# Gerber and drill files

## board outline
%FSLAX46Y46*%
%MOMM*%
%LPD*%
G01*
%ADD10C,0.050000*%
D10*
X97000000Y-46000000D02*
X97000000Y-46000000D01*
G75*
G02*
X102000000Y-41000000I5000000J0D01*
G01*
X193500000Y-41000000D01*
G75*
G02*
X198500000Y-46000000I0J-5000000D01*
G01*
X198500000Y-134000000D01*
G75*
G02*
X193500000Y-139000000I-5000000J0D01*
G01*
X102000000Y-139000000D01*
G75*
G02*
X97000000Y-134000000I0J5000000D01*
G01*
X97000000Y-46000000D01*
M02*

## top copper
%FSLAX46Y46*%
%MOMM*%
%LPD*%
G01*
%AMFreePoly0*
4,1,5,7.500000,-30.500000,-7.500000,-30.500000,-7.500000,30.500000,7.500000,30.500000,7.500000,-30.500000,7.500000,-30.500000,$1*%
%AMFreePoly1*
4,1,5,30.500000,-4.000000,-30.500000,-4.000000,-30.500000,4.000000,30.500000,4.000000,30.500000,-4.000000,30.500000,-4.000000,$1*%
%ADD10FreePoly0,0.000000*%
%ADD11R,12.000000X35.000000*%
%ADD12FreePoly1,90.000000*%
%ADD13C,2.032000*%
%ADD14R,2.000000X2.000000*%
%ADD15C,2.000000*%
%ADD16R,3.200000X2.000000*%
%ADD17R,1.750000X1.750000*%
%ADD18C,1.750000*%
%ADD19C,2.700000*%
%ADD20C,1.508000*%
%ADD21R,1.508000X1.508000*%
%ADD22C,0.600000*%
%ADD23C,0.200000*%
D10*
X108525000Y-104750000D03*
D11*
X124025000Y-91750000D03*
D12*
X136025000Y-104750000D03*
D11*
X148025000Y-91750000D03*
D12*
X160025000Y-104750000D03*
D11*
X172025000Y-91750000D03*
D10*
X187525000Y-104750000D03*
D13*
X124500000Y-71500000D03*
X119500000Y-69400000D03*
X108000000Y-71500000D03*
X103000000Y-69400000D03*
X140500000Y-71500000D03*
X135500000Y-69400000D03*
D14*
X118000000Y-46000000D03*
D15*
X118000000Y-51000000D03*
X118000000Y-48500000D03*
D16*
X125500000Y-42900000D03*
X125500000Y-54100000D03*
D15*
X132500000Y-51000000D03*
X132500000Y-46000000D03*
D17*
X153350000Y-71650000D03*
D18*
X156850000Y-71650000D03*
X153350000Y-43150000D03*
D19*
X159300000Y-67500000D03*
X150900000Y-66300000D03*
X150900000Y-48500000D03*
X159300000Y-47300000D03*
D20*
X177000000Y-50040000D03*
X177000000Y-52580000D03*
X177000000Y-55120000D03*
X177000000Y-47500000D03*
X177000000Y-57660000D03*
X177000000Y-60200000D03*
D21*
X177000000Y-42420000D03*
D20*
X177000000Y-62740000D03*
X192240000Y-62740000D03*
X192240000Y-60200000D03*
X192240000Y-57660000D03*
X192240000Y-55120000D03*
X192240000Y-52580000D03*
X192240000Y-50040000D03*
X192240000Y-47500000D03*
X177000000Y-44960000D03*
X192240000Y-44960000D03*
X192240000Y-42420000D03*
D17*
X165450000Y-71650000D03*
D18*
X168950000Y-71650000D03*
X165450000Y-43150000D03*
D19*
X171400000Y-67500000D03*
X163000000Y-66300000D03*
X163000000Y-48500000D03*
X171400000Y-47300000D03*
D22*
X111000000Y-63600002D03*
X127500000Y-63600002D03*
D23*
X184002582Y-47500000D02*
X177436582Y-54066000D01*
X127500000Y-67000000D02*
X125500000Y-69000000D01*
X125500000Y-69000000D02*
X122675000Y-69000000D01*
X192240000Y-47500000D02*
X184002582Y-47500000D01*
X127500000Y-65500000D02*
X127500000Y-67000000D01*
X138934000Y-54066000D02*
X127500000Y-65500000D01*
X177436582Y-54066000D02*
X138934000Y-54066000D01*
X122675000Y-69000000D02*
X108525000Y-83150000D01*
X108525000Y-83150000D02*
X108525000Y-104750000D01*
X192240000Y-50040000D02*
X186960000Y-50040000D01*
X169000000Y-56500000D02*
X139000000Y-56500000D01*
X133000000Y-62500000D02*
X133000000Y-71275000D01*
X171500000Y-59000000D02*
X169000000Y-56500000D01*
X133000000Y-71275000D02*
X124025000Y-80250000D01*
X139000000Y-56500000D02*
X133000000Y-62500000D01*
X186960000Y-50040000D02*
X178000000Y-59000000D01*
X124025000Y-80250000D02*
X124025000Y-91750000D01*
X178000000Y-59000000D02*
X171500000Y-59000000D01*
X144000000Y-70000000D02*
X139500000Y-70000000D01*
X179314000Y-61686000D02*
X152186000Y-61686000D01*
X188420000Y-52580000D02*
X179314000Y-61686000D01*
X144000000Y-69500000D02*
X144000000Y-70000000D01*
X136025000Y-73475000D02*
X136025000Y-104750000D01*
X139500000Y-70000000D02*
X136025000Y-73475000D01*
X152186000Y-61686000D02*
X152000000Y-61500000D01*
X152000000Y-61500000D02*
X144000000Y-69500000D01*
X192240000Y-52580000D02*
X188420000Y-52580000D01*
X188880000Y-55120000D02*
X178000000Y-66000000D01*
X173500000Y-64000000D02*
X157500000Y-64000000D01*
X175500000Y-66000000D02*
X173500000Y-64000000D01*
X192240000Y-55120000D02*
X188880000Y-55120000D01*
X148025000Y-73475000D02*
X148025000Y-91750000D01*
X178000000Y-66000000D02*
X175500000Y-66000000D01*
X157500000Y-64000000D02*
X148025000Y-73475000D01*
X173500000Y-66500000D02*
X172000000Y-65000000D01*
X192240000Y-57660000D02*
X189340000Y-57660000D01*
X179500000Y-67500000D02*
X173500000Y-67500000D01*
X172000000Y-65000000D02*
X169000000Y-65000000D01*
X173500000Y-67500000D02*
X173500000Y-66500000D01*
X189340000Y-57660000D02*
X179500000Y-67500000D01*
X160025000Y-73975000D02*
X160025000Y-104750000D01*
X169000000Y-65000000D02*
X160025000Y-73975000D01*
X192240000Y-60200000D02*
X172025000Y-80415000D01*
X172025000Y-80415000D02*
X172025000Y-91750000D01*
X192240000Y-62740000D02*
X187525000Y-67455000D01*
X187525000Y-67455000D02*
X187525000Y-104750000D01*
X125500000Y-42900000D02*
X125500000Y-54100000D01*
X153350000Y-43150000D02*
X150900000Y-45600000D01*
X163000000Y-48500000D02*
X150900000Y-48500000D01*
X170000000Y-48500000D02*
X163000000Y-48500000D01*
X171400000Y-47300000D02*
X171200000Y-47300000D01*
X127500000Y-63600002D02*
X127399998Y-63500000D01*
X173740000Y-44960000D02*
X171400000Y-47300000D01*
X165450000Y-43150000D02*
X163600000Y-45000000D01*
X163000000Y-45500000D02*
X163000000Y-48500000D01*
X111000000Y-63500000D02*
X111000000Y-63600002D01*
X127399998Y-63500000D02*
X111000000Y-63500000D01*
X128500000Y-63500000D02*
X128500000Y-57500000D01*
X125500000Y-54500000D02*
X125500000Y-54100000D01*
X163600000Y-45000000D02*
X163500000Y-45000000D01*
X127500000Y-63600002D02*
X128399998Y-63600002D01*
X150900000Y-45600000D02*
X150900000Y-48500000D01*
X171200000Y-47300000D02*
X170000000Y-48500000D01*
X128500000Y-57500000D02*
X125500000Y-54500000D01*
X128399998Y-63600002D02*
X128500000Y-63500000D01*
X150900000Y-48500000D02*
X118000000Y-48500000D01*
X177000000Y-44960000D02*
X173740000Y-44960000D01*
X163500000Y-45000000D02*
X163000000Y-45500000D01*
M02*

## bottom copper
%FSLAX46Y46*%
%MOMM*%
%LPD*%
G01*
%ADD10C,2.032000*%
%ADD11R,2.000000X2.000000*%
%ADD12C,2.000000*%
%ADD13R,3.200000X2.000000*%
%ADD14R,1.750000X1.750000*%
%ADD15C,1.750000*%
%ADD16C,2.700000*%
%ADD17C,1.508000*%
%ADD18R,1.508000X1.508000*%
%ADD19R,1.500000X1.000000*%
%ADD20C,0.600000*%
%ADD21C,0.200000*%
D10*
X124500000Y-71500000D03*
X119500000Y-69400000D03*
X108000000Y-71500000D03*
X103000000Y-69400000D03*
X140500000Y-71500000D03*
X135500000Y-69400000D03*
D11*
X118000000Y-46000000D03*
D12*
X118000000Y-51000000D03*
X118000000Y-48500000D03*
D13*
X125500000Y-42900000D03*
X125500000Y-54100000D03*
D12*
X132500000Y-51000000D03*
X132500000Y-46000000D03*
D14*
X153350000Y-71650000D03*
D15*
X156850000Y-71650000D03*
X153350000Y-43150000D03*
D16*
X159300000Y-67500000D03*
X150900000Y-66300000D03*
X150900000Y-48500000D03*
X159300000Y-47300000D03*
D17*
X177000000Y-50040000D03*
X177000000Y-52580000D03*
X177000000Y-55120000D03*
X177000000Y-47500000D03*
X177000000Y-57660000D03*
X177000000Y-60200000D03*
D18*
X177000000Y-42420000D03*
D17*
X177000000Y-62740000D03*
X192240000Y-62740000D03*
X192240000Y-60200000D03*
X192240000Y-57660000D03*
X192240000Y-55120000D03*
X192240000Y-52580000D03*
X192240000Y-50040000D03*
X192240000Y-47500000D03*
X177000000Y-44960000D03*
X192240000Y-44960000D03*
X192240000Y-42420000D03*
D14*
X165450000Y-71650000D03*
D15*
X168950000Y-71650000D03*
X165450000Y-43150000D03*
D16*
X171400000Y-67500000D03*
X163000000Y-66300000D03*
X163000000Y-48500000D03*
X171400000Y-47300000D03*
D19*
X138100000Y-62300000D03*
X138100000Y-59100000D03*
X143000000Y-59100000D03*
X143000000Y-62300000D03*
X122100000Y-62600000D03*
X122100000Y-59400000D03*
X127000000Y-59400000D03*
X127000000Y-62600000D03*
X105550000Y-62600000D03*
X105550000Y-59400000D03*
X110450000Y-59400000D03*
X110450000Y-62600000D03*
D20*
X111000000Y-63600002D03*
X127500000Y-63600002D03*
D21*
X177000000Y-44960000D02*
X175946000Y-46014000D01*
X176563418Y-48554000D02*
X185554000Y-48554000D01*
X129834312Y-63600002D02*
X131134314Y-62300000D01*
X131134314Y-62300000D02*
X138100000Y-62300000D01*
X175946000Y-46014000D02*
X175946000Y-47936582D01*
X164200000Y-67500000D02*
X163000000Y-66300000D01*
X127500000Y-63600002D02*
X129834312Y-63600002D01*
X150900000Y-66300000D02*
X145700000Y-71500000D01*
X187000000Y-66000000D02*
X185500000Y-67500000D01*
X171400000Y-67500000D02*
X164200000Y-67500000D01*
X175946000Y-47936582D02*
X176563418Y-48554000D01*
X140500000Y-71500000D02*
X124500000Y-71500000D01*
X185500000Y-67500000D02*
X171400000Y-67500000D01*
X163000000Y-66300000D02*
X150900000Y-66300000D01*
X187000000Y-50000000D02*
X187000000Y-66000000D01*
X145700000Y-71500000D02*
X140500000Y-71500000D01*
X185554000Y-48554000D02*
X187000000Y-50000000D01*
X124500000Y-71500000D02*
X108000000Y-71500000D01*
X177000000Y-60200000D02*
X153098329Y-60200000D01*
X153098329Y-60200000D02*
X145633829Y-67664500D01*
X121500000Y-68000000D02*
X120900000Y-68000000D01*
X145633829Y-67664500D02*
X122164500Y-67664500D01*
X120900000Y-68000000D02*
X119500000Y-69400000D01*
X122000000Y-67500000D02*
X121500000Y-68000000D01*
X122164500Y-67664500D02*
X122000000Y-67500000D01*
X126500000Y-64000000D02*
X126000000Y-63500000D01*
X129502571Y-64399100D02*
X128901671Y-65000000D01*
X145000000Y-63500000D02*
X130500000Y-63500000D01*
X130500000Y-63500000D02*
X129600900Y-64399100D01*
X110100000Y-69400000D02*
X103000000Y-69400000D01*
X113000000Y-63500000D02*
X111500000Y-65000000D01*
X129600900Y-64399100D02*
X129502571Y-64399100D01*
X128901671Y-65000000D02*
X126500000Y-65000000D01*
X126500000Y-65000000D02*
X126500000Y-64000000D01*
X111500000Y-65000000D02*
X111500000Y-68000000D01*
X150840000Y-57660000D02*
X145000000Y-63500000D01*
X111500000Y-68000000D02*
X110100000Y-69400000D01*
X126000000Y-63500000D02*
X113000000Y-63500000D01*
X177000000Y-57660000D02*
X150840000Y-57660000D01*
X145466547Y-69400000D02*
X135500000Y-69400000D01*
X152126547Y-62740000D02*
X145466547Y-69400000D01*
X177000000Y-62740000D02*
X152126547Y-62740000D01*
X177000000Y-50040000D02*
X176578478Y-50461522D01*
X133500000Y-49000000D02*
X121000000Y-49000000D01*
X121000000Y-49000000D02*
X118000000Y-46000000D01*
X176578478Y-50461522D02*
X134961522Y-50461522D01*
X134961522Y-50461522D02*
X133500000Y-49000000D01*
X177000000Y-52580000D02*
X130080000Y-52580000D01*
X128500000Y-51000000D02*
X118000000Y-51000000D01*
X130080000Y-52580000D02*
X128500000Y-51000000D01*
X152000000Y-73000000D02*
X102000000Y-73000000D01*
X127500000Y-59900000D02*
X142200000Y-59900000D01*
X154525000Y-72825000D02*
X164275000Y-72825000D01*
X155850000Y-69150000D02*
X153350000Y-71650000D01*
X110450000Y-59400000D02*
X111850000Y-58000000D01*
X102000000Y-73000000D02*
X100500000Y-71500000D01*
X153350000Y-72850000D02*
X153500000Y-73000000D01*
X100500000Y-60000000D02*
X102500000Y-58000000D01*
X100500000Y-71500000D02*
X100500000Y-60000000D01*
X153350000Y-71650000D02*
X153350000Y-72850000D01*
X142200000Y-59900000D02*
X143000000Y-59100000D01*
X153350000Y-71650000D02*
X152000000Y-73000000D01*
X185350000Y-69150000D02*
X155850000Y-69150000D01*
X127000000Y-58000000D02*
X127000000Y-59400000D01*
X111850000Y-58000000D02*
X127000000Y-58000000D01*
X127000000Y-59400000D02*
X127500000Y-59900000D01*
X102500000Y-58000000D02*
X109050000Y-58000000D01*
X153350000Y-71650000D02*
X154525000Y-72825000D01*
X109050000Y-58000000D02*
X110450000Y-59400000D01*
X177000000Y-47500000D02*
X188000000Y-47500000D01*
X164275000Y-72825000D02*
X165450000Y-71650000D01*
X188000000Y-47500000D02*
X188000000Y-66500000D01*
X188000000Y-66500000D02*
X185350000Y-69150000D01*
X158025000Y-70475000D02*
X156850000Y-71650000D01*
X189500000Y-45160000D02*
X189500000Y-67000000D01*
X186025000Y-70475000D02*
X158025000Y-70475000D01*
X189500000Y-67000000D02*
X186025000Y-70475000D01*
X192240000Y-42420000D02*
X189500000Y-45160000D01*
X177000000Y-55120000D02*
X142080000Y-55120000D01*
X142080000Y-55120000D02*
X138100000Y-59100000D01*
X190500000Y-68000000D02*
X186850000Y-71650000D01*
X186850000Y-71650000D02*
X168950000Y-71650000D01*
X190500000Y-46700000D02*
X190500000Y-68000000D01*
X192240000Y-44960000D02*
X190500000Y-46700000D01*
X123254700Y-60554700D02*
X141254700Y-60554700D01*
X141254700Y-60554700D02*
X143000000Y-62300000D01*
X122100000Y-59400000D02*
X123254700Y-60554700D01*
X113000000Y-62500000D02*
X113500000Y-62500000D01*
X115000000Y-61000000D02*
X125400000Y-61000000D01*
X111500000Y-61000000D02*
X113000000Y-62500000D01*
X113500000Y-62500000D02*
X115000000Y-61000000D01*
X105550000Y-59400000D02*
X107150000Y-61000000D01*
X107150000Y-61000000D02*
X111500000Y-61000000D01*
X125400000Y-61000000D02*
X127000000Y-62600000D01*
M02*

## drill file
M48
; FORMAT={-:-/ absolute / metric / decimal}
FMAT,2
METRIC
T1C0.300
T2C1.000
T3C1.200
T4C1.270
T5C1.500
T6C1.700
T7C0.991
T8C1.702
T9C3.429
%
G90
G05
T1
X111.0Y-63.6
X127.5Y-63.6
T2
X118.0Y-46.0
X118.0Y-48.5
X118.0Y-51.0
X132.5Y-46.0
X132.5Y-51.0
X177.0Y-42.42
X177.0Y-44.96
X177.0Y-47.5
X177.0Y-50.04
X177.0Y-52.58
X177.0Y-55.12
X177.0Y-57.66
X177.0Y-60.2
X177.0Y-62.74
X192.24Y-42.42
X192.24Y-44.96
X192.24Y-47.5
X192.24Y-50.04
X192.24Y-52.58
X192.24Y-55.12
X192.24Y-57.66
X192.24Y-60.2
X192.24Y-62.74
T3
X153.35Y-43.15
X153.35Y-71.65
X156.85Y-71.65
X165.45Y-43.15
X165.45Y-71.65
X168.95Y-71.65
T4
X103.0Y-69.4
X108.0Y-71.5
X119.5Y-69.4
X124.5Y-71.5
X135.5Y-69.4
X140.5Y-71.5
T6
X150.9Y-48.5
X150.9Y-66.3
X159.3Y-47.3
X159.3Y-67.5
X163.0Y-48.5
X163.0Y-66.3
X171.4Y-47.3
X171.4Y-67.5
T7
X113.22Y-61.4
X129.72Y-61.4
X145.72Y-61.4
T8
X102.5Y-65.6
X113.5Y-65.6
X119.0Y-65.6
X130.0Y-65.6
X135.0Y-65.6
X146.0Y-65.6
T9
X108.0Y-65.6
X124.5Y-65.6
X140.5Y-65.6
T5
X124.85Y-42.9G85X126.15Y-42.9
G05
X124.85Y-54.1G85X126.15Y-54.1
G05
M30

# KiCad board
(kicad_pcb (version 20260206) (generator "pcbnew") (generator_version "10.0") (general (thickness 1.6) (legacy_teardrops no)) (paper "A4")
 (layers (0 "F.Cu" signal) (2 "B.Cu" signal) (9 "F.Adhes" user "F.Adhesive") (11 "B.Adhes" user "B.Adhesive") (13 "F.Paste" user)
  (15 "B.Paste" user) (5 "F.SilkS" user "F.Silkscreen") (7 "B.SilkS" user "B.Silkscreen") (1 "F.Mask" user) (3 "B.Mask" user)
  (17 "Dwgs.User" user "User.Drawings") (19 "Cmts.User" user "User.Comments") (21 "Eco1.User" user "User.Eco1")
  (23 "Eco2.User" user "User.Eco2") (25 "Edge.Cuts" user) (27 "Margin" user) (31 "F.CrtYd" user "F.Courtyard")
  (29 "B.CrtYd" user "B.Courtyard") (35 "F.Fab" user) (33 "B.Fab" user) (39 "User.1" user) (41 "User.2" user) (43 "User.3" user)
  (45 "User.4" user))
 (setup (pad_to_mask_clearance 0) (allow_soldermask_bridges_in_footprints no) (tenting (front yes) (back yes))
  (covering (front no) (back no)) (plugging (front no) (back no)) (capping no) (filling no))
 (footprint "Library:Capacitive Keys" (layer "F.Cu") (at 139.025 60.25)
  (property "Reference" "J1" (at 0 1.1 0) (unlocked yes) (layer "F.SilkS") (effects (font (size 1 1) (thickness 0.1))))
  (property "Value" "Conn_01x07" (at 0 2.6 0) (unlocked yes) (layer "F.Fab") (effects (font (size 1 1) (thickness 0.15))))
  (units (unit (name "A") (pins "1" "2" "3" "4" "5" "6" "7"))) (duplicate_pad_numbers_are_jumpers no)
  (pad "1" smd custom (at -30.5 44.5) (size 15 61) (layers "F.Cu" "F.Mask") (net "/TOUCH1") (options (clearance outline) (anchor rect))
   (primitives))
  (pad "2" smd rect (at -15 31.5) (size 12 35) (layers "F.Cu" "F.Mask") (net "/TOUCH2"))
  (pad "3" smd custom (at -3 44.5 90) (size 61 8) (layers "F.Cu" "F.Mask") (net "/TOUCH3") (options (clearance outline) (anchor rect))
   (primitives))
  (pad "4" smd rect (at 9 31.5) (size 12 35) (layers "F.Cu" "F.Mask") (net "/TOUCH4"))
  (pad "5" smd custom (at 21 44.5 90) (size 61 8) (layers "F.Cu" "F.Mask") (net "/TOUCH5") (options (clearance outline) (anchor rect))
   (primitives))
  (pad "6" smd rect (at 33 31.5) (size 12 35) (layers "F.Cu" "F.Mask") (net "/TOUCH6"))
  (pad "7" smd custom (at 48.5 44.5) (size 15 61) (layers "F.Cu" "F.Mask") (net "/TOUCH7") (options (clearance outline) (anchor rect))
   (primitives)))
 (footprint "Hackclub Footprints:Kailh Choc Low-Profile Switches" (layer "F.Cu") (at 124.5 65.6)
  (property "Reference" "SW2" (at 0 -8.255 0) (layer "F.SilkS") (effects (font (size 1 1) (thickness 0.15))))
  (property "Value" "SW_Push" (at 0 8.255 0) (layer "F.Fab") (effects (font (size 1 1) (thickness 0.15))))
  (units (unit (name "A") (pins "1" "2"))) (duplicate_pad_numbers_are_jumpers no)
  (pad "" np_thru_hole circle (at -5.5 0) (size 1.7018 1.7018) (drill 1.7018) (layers "*.Cu" "*.Mask"))
  (pad "" np_thru_hole circle (at 0 0) (size 3.429 3.429) (drill 3.429) (layers "*.Cu" "*.Mask"))
  (pad "" np_thru_hole circle (at 5.22 -4.2) (size 0.9906 0.9906) (drill 0.9906) (layers "*.Cu" "*.Mask"))
  (pad "" np_thru_hole circle (at 5.5 0) (size 1.7018 1.7018) (drill 1.7018) (layers "*.Cu" "*.Mask"))
  (pad "1" thru_hole circle (at 0 5.9) (size 2.032 2.032) (drill 1.27) (layers "*.Cu" "*.Mask") (remove_unused_layers no) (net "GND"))
  (pad "2" thru_hole circle (at -5 3.8) (size 2.032 2.032) (drill 1.27) (layers "*.Cu" "*.Mask") (remove_unused_layers no) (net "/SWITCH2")))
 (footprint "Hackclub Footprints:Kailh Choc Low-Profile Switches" (layer "F.Cu") (at 108 65.6)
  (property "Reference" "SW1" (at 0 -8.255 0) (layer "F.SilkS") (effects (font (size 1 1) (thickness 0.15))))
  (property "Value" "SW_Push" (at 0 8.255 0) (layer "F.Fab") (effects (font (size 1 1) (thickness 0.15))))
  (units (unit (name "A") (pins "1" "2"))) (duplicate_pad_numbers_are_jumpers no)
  (pad "" np_thru_hole circle (at -5.5 0) (size 1.7018 1.7018) (drill 1.7018) (layers "*.Cu" "*.Mask"))
  (pad "" np_thru_hole circle (at 0 0) (size 3.429 3.429) (drill 3.429) (layers "*.Cu" "*.Mask"))
  (pad "" np_thru_hole circle (at 5.22 -4.2) (size 0.9906 0.9906) (drill 0.9906) (layers "*.Cu" "*.Mask"))
  (pad "" np_thru_hole circle (at 5.5 0) (size 1.7018 1.7018) (drill 1.7018) (layers "*.Cu" "*.Mask"))
  (pad "1" thru_hole circle (at 0 5.9) (size 2.032 2.032) (drill 1.27) (layers "*.Cu" "*.Mask") (remove_unused_layers no) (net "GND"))
  (pad "2" thru_hole circle (at -5 3.8) (size 2.032 2.032) (drill 1.27) (layers "*.Cu" "*.Mask") (remove_unused_layers no) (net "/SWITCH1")))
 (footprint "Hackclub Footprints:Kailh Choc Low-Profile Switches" (layer "F.Cu") (at 140.5 65.6)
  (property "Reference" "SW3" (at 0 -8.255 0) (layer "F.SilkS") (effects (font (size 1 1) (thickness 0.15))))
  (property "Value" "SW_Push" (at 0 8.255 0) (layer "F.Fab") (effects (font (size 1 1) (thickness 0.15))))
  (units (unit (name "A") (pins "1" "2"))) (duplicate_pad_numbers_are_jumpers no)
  (pad "" np_thru_hole circle (at -5.5 0) (size 1.7018 1.7018) (drill 1.7018) (layers "*.Cu" "*.Mask"))
  (pad "" np_thru_hole circle (at 0 0) (size 3.429 3.429) (drill 3.429) (layers "*.Cu" "*.Mask"))
  (pad "" np_thru_hole circle (at 5.22 -4.2) (size 0.9906 0.9906) (drill 0.9906) (layers "*.Cu" "*.Mask"))
  (pad "" np_thru_hole circle (at 5.5 0) (size 1.7018 1.7018) (drill 1.7018) (layers "*.Cu" "*.Mask"))
  (pad "1" thru_hole circle (at 0 5.9) (size 2.032 2.032) (drill 1.27) (layers "*.Cu" "*.Mask") (remove_unused_layers no) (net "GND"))
  (pad "2" thru_hole circle (at -5 3.8) (size 2.032 2.032) (drill 1.27) (layers "*.Cu" "*.Mask") (remove_unused_layers no) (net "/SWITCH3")))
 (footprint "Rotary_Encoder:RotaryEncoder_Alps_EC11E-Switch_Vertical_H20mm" (layer "F.Cu") (at 118 46)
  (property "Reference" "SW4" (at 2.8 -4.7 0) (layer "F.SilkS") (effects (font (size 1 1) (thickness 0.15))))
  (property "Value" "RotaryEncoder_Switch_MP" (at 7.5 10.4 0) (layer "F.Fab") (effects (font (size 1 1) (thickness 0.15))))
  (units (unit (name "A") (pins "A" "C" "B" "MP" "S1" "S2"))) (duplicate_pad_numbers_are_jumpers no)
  (pad "A" thru_hole rect (at 0 0) (size 2 2) (drill 1) (layers "*.Cu" "*.Mask") (remove_unused_layers no) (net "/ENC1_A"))
  (pad "B" thru_hole circle (at 0 5) (size 2 2) (drill 1) (layers "*.Cu" "*.Mask") (remove_unused_layers no) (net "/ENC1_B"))
  (pad "C" thru_hole circle (at 0 2.5) (size 2 2) (drill 1) (layers "*.Cu" "*.Mask") (remove_unused_layers no) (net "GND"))
  (pad "MP" thru_hole rect (at 7.5 -3.1) (size 3.2 2) (drill oval 2.8 1.5) (layers "*.Cu" "*.Mask") (remove_unused_layers no) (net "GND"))
  (pad "MP" thru_hole rect (at 7.5 8.1) (size 3.2 2) (drill oval 2.8 1.5) (layers "*.Cu" "*.Mask") (remove_unused_layers no) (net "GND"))
  (pad "S1" thru_hole circle (at 14.5 5) (size 2 2) (drill 1) (layers "*.Cu" "*.Mask") (remove_unused_layers no)
   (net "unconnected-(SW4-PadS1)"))
  (pad "S2" thru_hole circle (at 14.5 0) (size 2 2) (drill 1) (layers "*.Cu" "*.Mask") (remove_unused_layers no)
   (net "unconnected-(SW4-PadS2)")))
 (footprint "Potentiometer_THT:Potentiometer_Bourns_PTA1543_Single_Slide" (layer "F.Cu") (at 153.35 71.65 90)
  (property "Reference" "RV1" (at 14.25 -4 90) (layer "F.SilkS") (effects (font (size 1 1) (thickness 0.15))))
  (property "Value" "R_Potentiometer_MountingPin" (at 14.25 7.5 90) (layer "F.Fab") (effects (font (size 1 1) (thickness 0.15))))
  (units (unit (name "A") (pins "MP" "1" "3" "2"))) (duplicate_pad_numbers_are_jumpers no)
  (pad "1" thru_hole rect (at 0 0 90) (size 1.75 1.75) (drill 1.2) (layers "*.Cu" "*.Mask") (remove_unused_layers no) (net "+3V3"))
  (pad "2" thru_hole circle (at 0 3.5 90) (size 1.75 1.75) (drill 1.2) (layers "*.Cu" "*.Mask") (remove_unused_layers no) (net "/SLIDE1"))
  (pad "3" thru_hole circle (at 28.5 0 90) (size 1.75 1.75) (drill 1.2) (layers "*.Cu" "*.Mask") (remove_unused_layers no) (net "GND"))
  (pad "MP" thru_hole circle (at 4.15 5.95 90) (size 2.7 2.7) (drill 1.7) (layers "*.Cu" "*.Mask") (remove_unused_layers no) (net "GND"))
  (pad "MP" thru_hole circle (at 5.35 -2.45 90) (size 2.7 2.7) (drill 1.7) (layers "*.Cu" "*.Mask") (remove_unused_layers no) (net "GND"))
  (pad "MP" thru_hole circle (at 23.15 -2.45 90) (size 2.7 2.7) (drill 1.7) (layers "*.Cu" "*.Mask") (remove_unused_layers no) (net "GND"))
  (pad "MP" thru_hole circle (at 24.35 5.95 90) (size 2.7 2.7) (drill 1.7) (layers "*.Cu" "*.Mask") (remove_unused_layers no) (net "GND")))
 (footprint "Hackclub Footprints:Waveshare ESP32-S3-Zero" (layer "F.Cu") (at 184.62 52.58)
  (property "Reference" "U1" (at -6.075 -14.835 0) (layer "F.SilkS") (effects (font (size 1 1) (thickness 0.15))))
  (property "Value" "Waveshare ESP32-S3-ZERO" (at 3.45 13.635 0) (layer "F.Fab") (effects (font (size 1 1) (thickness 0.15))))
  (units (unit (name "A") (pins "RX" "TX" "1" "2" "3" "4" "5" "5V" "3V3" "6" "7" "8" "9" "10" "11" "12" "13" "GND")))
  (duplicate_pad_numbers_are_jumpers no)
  (pad "1" thru_hole circle (at -7.62 -2.54) (size 1.508 1.508) (drill 1) (layers "*.Cu" "*.Mask") (remove_unused_layers no) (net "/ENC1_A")
   (solder_mask_margin 0.102))
  (pad "2" thru_hole circle (at -7.62 0) (size 1.508 1.508) (drill 1) (layers "*.Cu" "*.Mask") (remove_unused_layers no) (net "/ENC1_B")
   (solder_mask_margin 0.102))
  (pad "3" thru_hole circle (at -7.62 2.54) (size 1.508 1.508) (drill 1) (layers "*.Cu" "*.Mask") (remove_unused_layers no) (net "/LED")
   (solder_mask_margin 0.102))
  (pad "3V3" thru_hole circle (at -7.62 -5.08) (size 1.508 1.508) (drill 1) (layers "*.Cu" "*.Mask") (remove_unused_layers no) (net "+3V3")
   (solder_mask_margin 0.102))
  (pad "4" thru_hole circle (at -7.62 5.08) (size 1.508 1.508) (drill 1) (layers "*.Cu" "*.Mask") (remove_unused_layers no) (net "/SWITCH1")
   (solder_mask_margin 0.102))
  (pad "5" thru_hole circle (at -7.62 7.62) (size 1.508 1.508) (drill 1) (layers "*.Cu" "*.Mask") (remove_unused_layers no) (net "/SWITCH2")
   (solder_mask_margin 0.102))
  (pad "5V" thru_hole rect (at -7.62 -10.16) (size 1.508 1.508) (drill 1) (layers "*.Cu" "*.Mask") (remove_unused_layers no) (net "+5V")
   (solder_mask_margin 0.102))
  (pad "6" thru_hole circle (at -7.62 10.16) (size 1.508 1.508) (drill 1) (layers "*.Cu" "*.Mask") (remove_unused_layers no)
   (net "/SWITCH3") (solder_mask_margin 0.102))
  (pad "7" thru_hole circle (at 7.62 10.16) (size 1.508 1.508) (drill 1) (layers "*.Cu" "*.Mask") (remove_unused_layers no) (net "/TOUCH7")
   (solder_mask_margin 0.102))
  (pad "8" thru_hole circle (at 7.62 7.62) (size 1.508 1.508) (drill 1) (layers "*.Cu" "*.Mask") (remove_unused_layers no) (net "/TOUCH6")
   (solder_mask_margin 0.102))
  (pad "9" thru_hole circle (at 7.62 5.08) (size 1.508 1.508) (drill 1) (layers "*.Cu" "*.Mask") (remove_unused_layers no) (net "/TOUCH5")
   (solder_mask_margin 0.102))
  (pad "10" thru_hole circle (at 7.62 2.54) (size 1.508 1.508) (drill 1) (layers "*.Cu" "*.Mask") (remove_unused_layers no) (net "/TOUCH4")
   (solder_mask_margin 0.102))
  (pad "11" thru_hole circle (at 7.62 0) (size 1.508 1.508) (drill 1) (layers "*.Cu" "*.Mask") (remove_unused_layers no) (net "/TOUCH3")
   (solder_mask_margin 0.102))
  (pad "12" thru_hole circle (at 7.62 -2.54) (size 1.508 1.508) (drill 1) (layers "*.Cu" "*.Mask") (remove_unused_layers no) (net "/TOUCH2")
   (solder_mask_margin 0.102))
  (pad "13" thru_hole circle (at 7.62 -5.08) (size 1.508 1.508) (drill 1) (layers "*.Cu" "*.Mask") (remove_unused_layers no) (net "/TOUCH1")
   (solder_mask_margin 0.102))
  (pad "GND" thru_hole circle (at -7.62 -7.62) (size 1.508 1.508) (drill 1) (layers "*.Cu" "*.Mask") (remove_unused_layers no) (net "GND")
   (solder_mask_margin 0.102))
  (pad "RX" thru_hole circle (at 7.62 -7.62) (size 1.508 1.508) (drill 1) (layers "*.Cu" "*.Mask") (remove_unused_layers no) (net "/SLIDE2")
   (solder_mask_margin 0.102))
  (pad "TX" thru_hole circle (at 7.62 -10.16) (size 1.508 1.508) (drill 1) (layers "*.Cu" "*.Mask") (remove_unused_layers no)
   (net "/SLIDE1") (solder_mask_margin 0.102)))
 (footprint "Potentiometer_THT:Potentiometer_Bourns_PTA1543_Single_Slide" (layer "F.Cu") (at 165.45 71.65 90)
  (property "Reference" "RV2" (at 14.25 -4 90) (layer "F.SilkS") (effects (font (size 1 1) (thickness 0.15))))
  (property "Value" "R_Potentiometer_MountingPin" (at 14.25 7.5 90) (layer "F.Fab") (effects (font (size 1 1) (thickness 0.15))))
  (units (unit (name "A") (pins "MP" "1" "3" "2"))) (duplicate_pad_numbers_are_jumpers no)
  (pad "1" thru_hole rect (at 0 0 90) (size 1.75 1.75) (drill 1.2) (layers "*.Cu" "*.Mask") (remove_unused_layers no) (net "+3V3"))
  (pad "2" thru_hole circle (at 0 3.5 90) (size 1.75 1.75) (drill 1.2) (layers "*.Cu" "*.Mask") (remove_unused_layers no) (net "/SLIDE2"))
  (pad "3" thru_hole circle (at 28.5 0 90) (size 1.75 1.75) (drill 1.2) (layers "*.Cu" "*.Mask") (remove_unused_layers no) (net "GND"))
  (pad "MP" thru_hole circle (at 4.15 5.95 90) (size 2.7 2.7) (drill 1.7) (layers "*.Cu" "*.Mask") (remove_unused_layers no) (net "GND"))
  (pad "MP" thru_hole circle (at 5.35 -2.45 90) (size 2.7 2.7) (drill 1.7) (layers "*.Cu" "*.Mask") (remove_unused_layers no) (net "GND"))
  (pad "MP" thru_hole circle (at 23.15 -2.45 90) (size 2.7 2.7) (drill 1.7) (layers "*.Cu" "*.Mask") (remove_unused_layers no) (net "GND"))
  (pad "MP" thru_hole circle (at 24.35 5.95 90) (size 2.7 2.7) (drill 1.7) (layers "*.Cu" "*.Mask") (remove_unused_layers no) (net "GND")))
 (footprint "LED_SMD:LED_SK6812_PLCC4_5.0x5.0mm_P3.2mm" (layer "B.Cu") (at 140.55 60.7)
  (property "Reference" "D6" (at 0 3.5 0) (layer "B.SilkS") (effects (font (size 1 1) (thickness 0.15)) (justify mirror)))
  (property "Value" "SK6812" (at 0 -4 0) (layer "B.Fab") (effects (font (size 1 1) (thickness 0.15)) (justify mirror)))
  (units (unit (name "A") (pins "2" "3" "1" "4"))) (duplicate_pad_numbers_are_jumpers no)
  (pad "1" smd rect (at -2.45 1.6 180) (size 1.5 1) (layers "B.Cu" "B.Mask" "B.Paste") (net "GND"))
  (pad "2" smd rect (at -2.45 -1.6 180) (size 1.5 1) (layers "B.Cu" "B.Mask" "B.Paste") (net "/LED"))
  (pad "3" smd rect (at 2.45 -1.6 180) (size 1.5 1) (layers "B.Cu" "B.Mask" "B.Paste") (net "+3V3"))
  (pad "4" smd rect (at 2.45 1.6 180) (size 1.5 1) (layers "B.Cu" "B.Mask" "B.Paste") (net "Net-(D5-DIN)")))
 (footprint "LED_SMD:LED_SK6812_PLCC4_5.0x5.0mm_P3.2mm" (layer "B.Cu") (at 124.55 61)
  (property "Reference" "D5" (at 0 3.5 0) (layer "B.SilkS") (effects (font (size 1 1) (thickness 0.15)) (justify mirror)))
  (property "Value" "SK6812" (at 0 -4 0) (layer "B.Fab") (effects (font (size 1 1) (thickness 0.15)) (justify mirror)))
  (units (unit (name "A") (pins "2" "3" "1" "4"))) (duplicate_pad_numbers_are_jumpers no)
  (pad "1" smd rect (at -2.45 1.6 180) (size 1.5 1) (layers "B.Cu" "B.Mask" "B.Paste") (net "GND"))
  (pad "2" smd rect (at -2.45 -1.6 180) (size 1.5 1) (layers "B.Cu" "B.Mask" "B.Paste") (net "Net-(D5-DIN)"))
  (pad "3" smd rect (at 2.45 -1.6 180) (size 1.5 1) (layers "B.Cu" "B.Mask" "B.Paste") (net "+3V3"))
  (pad "4" smd rect (at 2.45 1.6 180) (size 1.5 1) (layers "B.Cu" "B.Mask" "B.Paste") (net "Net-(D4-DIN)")))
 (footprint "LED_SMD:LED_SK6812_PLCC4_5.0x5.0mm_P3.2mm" (layer "B.Cu") (at 108 61)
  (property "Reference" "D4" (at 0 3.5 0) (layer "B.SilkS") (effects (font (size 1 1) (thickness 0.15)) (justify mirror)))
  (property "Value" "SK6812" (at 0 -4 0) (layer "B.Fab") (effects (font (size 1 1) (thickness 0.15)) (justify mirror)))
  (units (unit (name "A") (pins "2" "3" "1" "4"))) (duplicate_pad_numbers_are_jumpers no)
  (pad "1" smd rect (at -2.45 1.6 180) (size 1.5 1) (layers "B.Cu" "B.Mask" "B.Paste") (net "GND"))
  (pad "2" smd rect (at -2.45 -1.6 180) (size 1.5 1) (layers "B.Cu" "B.Mask" "B.Paste") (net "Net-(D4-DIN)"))
  (pad "3" smd rect (at 2.45 -1.6 180) (size 1.5 1) (layers "B.Cu" "B.Mask" "B.Paste") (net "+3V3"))
  (pad "4" smd rect (at 2.45 1.6 180) (size 1.5 1) (layers "B.Cu" "B.Mask" "B.Paste") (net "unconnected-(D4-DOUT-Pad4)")))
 (gr_rect (start 97 41) (end 198.5 139) (radius 5) (stroke (width 0.05) (type solid)) (fill no) (layer "Edge.Cuts"))
 (segment (start 184.002582 47.5) (end 177.436582 54.066) (width 0.2) (layer "F.Cu") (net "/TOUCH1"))
 (segment (start 127.5 67) (end 125.5 69) (width 0.2) (layer "F.Cu") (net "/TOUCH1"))
 (segment (start 125.5 69) (end 122.675 69) (width 0.2) (layer "F.Cu") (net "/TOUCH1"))
 (segment (start 192.24 47.5) (end 184.002582 47.5) (width 0.2) (layer "F.Cu") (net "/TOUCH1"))
 (segment (start 127.5 65.5) (end 127.5 67) (width 0.2) (layer "F.Cu") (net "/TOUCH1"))
 (segment (start 138.934 54.066) (end 127.5 65.5) (width 0.2) (layer "F.Cu") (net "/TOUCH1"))
 (segment (start 177.436582 54.066) (end 138.934 54.066) (width 0.2) (layer "F.Cu") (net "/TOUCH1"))
 (segment (start 122.675 69) (end 108.525 83.15) (width 0.2) (layer "F.Cu") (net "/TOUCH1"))
 (segment (start 108.525 83.15) (end 108.525 104.75) (width 0.2) (layer "F.Cu") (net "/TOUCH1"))
 (segment (start 192.24 50.04) (end 186.96 50.04) (width 0.2) (layer "F.Cu") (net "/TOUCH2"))
 (segment (start 169 56.5) (end 139 56.5) (width 0.2) (layer "F.Cu") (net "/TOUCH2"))
 (segment (start 133 62.5) (end 133 71.275) (width 0.2) (layer "F.Cu") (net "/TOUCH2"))
 (segment (start 171.5 59) (end 169 56.5) (width 0.2) (layer "F.Cu") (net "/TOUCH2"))
 (segment (start 133 71.275) (end 124.025 80.25) (width 0.2) (layer "F.Cu") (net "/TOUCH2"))
 (segment (start 139 56.5) (end 133 62.5) (width 0.2) (layer "F.Cu") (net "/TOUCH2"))
 (segment (start 186.96 50.04) (end 178 59) (width 0.2) (layer "F.Cu") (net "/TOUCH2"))
 (segment (start 124.025 80.25) (end 124.025 91.75) (width 0.2) (layer "F.Cu") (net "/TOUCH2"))
 (segment (start 178 59) (end 171.5 59) (width 0.2) (layer "F.Cu") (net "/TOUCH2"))
 (segment (start 144 70) (end 139.5 70) (width 0.2) (layer "F.Cu") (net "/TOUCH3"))
 (segment (start 179.314 61.686) (end 152.186 61.686) (width 0.2) (layer "F.Cu") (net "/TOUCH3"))
 (segment (start 188.42 52.58) (end 179.314 61.686) (width 0.2) (layer "F.Cu") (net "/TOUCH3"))
 (segment (start 144 69.5) (end 144 70) (width 0.2) (layer "F.Cu") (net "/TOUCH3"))
 (segment (start 136.025 73.475) (end 136.025 104.75) (width 0.2) (layer "F.Cu") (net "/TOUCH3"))
 (segment (start 139.5 70) (end 136.025 73.475) (width 0.2) (layer "F.Cu") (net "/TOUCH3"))
 (segment (start 152.186 61.686) (end 152 61.5) (width 0.2) (layer "F.Cu") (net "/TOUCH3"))
 (segment (start 152 61.5) (end 144 69.5) (width 0.2) (layer "F.Cu") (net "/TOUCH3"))
 (segment (start 192.24 52.58) (end 188.42 52.58) (width 0.2) (layer "F.Cu") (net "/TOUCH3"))
 (segment (start 188.88 55.12) (end 178 66) (width 0.2) (layer "F.Cu") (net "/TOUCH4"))
 (segment (start 173.5 64) (end 157.5 64) (width 0.2) (layer "F.Cu") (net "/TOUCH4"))
 (segment (start 175.5 66) (end 173.5 64) (width 0.2) (layer "F.Cu") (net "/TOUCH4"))
 (segment (start 192.24 55.12) (end 188.88 55.12) (width 0.2) (layer "F.Cu") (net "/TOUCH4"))
 (segment (start 148.025 73.475) (end 148.025 91.75) (width 0.2) (layer "F.Cu") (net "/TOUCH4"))
 (segment (start 178 66) (end 175.5 66) (width 0.2) (layer "F.Cu") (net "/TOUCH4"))
 (segment (start 157.5 64) (end 148.025 73.475) (width 0.2) (layer "F.Cu") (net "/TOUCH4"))
 (segment (start 173.5 66.5) (end 172 65) (width 0.2) (layer "F.Cu") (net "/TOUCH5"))
 (segment (start 192.24 57.66) (end 189.34 57.66) (width 0.2) (layer "F.Cu") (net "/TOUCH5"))
 (segment (start 179.5 67.5) (end 173.5 67.5) (width 0.2) (layer "F.Cu") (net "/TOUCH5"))
 (segment (start 172 65) (end 169 65) (width 0.2) (layer "F.Cu") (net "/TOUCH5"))
 (segment (start 173.5 67.5) (end 173.5 66.5) (width 0.2) (layer "F.Cu") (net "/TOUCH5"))
 (segment (start 189.34 57.66) (end 179.5 67.5) (width 0.2) (layer "F.Cu") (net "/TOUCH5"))
 (segment (start 160.025 73.975) (end 160.025 104.75) (width 0.2) (layer "F.Cu") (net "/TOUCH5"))
 (segment (start 169 65) (end 160.025 73.975) (width 0.2) (layer "F.Cu") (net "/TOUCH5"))
 (segment (start 192.24 60.2) (end 172.025 80.415) (width 0.2) (layer "F.Cu") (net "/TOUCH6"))
 (segment (start 172.025 80.415) (end 172.025 91.75) (width 0.2) (layer "F.Cu") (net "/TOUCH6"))
 (segment (start 192.24 62.74) (end 187.525 67.455) (width 0.2) (layer "F.Cu") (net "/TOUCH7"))
 (segment (start 187.525 67.455) (end 187.525 104.75) (width 0.2) (layer "F.Cu") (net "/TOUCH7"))
 (segment (start 125.5 42.9) (end 125.5 54.1) (width 0.2) (layer "F.Cu") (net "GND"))
 (segment (start 153.35 43.15) (end 150.9 45.6) (width 0.2) (layer "F.Cu") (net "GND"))
 (segment (start 163 48.5) (end 150.9 48.5) (width 0.2) (layer "F.Cu") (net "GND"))
 (segment (start 170 48.5) (end 163 48.5) (width 0.2) (layer "F.Cu") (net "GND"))
 (segment (start 171.4 47.3) (end 171.2 47.3) (width 0.2) (layer "F.Cu") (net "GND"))
 (segment (start 127.5 63.600002) (end 127.399998 63.5) (width 0.2) (layer "F.Cu") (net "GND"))
 (segment (start 173.74 44.96) (end 171.4 47.3) (width 0.2) (layer "F.Cu") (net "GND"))
 (segment (start 165.45 43.15) (end 163.6 45) (width 0.2) (layer "F.Cu") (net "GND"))
 (segment (start 163 45.5) (end 163 48.5) (width 0.2) (layer "F.Cu") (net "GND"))
 (segment (start 111 63.5) (end 111 63.600002) (width 0.2) (layer "F.Cu") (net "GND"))
 (segment (start 127.399998 63.5) (end 111 63.5) (width 0.2) (layer "F.Cu") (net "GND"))
 (segment (start 128.5 63.5) (end 128.5 57.5) (width 0.2) (layer "F.Cu") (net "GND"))
 (segment (start 125.5 54.5) (end 125.5 54.1) (width 0.2) (layer "F.Cu") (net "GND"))
 (segment (start 163.6 45) (end 163.5 45) (width 0.2) (layer "F.Cu") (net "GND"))
 (segment (start 127.5 63.600002) (end 128.399998 63.600002) (width 0.2) (layer "F.Cu") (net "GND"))
 (segment (start 150.9 45.6) (end 150.9 48.5) (width 0.2) (layer "F.Cu") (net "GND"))
 (segment (start 171.2 47.3) (end 170 48.5) (width 0.2) (layer "F.Cu") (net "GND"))
 (segment (start 128.5 57.5) (end 125.5 54.5) (width 0.2) (layer "F.Cu") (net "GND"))
 (segment (start 128.399998 63.600002) (end 128.5 63.5) (width 0.2) (layer "F.Cu") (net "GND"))
 (segment (start 150.9 48.5) (end 118 48.5) (width 0.2) (layer "F.Cu") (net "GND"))
 (segment (start 177 44.96) (end 173.74 44.96) (width 0.2) (layer "F.Cu") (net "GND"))
 (segment (start 163.5 45) (end 163 45.5) (width 0.2) (layer "F.Cu") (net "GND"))
 (via (at 111 63.600002) (size 0.6) (drill 0.3) (layers "F.Cu" "B.Cu") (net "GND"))
 (via (at 127.5 63.600002) (size 0.6) (drill 0.3) (layers "F.Cu" "B.Cu") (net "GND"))
 (segment (start 177 44.96) (end 175.946 46.014) (width 0.2) (layer "B.Cu") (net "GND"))
 (segment (start 176.563418 48.554) (end 185.554 48.554) (width 0.2) (layer "B.Cu") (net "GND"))
 (segment (start 129.834312 63.600002) (end 131.134314 62.3) (width 0.2) (layer "B.Cu") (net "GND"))
 (segment (start 131.134314 62.3) (end 138.1 62.3) (width 0.2) (layer "B.Cu") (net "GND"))
 (segment (start 175.946 46.014) (end 175.946 47.936582) (width 0.2) (layer "B.Cu") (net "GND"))
 (segment (start 164.2 67.5) (end 163 66.3) (width 0.2) (layer "B.Cu") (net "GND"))
 (segment (start 127.5 63.600002) (end 129.834312 63.600002) (width 0.2) (layer "B.Cu") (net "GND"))
 (segment (start 150.9 66.3) (end 145.7 71.5) (width 0.2) (layer "B.Cu") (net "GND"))
 (segment (start 187 66) (end 185.5 67.5) (width 0.2) (layer "B.Cu") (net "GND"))
 (segment (start 171.4 67.5) (end 164.2 67.5) (width 0.2) (layer "B.Cu") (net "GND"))
 (segment (start 175.946 47.936582) (end 176.563418 48.554) (width 0.2) (layer "B.Cu") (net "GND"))
 (segment (start 140.5 71.5) (end 124.5 71.5) (width 0.2) (layer "B.Cu") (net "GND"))
 (segment (start 185.5 67.5) (end 171.4 67.5) (width 0.2) (layer "B.Cu") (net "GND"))
 (segment (start 163 66.3) (end 150.9 66.3) (width 0.2) (layer "B.Cu") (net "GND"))
 (segment (start 187 50) (end 187 66) (width 0.2) (layer "B.Cu") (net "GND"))
 (segment (start 145.7 71.5) (end 140.5 71.5) (width 0.2) (layer "B.Cu") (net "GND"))
 (segment (start 185.554 48.554) (end 187 50) (width 0.2) (layer "B.Cu") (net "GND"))
 (segment (start 124.5 71.5) (end 108 71.5) (width 0.2) (layer "B.Cu") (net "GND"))
 (segment (start 177 60.2) (end 153.098329 60.2) (width 0.2) (layer "B.Cu") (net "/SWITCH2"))
 (segment (start 153.098329 60.2) (end 145.633829 67.6645) (width 0.2) (layer "B.Cu") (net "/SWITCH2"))
 (segment (start 121.5 68) (end 120.9 68) (width 0.2) (layer "B.Cu") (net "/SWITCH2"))
 (segment (start 145.633829 67.6645) (end 122.1645 67.6645) (width 0.2) (layer "B.Cu") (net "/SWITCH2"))
 (segment (start 120.9 68) (end 119.5 69.4) (width 0.2) (layer "B.Cu") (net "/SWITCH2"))
 (segment (start 122 67.5) (end 121.5 68) (width 0.2) (layer "B.Cu") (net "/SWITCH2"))
 (segment (start 122.1645 67.6645) (end 122 67.5) (width 0.2) (layer "B.Cu") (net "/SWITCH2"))
 (segment (start 126.5 64) (end 126 63.5) (width 0.2) (layer "B.Cu") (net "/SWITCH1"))
 (segment (start 129.502571 64.3991) (end 128.901671 65) (width 0.2) (layer "B.Cu") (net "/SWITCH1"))
 (segment (start 145 63.5) (end 130.5 63.5) (width 0.2) (layer "B.Cu") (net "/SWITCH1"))
 (segment (start 130.5 63.5) (end 129.6009 64.3991) (width 0.2) (layer "B.Cu") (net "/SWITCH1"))
 (segment (start 110.1 69.4) (end 103 69.4) (width 0.2) (layer "B.Cu") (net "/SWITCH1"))
 (segment (start 113 63.5) (end 111.5 65) (width 0.2) (layer "B.Cu") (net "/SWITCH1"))
 (segment (start 129.6009 64.3991) (end 129.502571 64.3991) (width 0.2) (layer "B.Cu") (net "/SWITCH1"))
 (segment (start 128.901671 65) (end 126.5 65) (width 0.2) (layer "B.Cu") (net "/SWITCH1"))
 (segment (start 126.5 65) (end 126.5 64) (width 0.2) (layer "B.Cu") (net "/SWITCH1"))
 (segment (start 111.5 65) (end 111.5 68) (width 0.2) (layer "B.Cu") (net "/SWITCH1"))
 (segment (start 150.84 57.66) (end 145 63.5) (width 0.2) (layer "B.Cu") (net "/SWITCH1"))
 (segment (start 111.5 68) (end 110.1 69.4) (width 0.2) (layer "B.Cu") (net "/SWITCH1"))
 (segment (start 126 63.5) (end 113 63.5) (width 0.2) (layer "B.Cu") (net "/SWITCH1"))
 (segment (start 177 57.66) (end 150.84 57.66) (width 0.2) (layer "B.Cu") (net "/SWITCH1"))
 (segment (start 145.466547 69.4) (end 135.5 69.4) (width 0.2) (layer "B.Cu") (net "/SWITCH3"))
 (segment (start 152.126547 62.74) (end 145.466547 69.4) (width 0.2) (layer "B.Cu") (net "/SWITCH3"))
 (segment (start 177 62.74) (end 152.126547 62.74) (width 0.2) (layer "B.Cu") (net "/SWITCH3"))
 (segment (start 177 50.04) (end 176.578478 50.461522) (width 0.2) (layer "B.Cu") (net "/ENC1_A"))
 (segment (start 133.5 49) (end 121 49) (width 0.2) (layer "B.Cu") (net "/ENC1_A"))
 (segment (start 121 49) (end 118 46) (width 0.2) (layer "B.Cu") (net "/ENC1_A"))
 (segment (start 176.578478 50.461522) (end 134.961522 50.461522) (width 0.2) (layer "B.Cu") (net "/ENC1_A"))
 (segment (start 134.961522 50.461522) (end 133.5 49) (width 0.2) (layer "B.Cu") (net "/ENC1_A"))
 (segment (start 177 52.58) (end 130.08 52.58) (width 0.2) (layer "B.Cu") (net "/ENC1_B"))
 (segment (start 128.5 51) (end 118 51) (width 0.2) (layer "B.Cu") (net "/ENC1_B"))
 (segment (start 130.08 52.58) (end 128.5 51) (width 0.2) (layer "B.Cu") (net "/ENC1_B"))
 (segment (start 152 73) (end 102 73) (width 0.2) (layer "B.Cu") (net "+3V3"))
 (segment (start 127.5 59.9) (end 142.2 59.9) (width 0.2) (layer "B.Cu") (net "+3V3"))
 (segment (start 154.525 72.825) (end 164.275 72.825) (width 0.2) (layer "B.Cu") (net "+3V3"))
 (segment (start 155.85 69.15) (end 153.35 71.65) (width 0.2) (layer "B.Cu") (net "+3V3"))
 (segment (start 110.45 59.4) (end 111.85 58) (width 0.2) (layer "B.Cu") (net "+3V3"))
 (segment (start 102 73) (end 100.5 71.5) (width 0.2) (layer "B.Cu") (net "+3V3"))
 (segment (start 153.35 72.85) (end 153.5 73) (width 0.2) (layer "B.Cu") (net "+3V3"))
 (segment (start 100.5 60) (end 102.5 58) (width 0.2) (layer "B.Cu") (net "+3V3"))
 (segment (start 100.5 71.5) (end 100.5 60) (width 0.2) (layer "B.Cu") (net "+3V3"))
 (segment (start 153.35 71.65) (end 153.35 72.85) (width 0.2) (layer "B.Cu") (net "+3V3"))
 (segment (start 142.2 59.9) (end 143 59.1) (width 0.2) (layer "B.Cu") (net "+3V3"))
 (segment (start 153.35 71.65) (end 152 73) (width 0.2) (layer "B.Cu") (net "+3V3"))
 (segment (start 185.35 69.15) (end 155.85 69.15) (width 0.2) (layer "B.Cu") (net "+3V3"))
 (segment (start 127 58) (end 127 59.4) (width 0.2) (layer "B.Cu") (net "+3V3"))
 (segment (start 111.85 58) (end 127 58) (width 0.2) (layer "B.Cu") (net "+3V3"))
 (segment (start 127 59.4) (end 127.5 59.9) (width 0.2) (layer "B.Cu") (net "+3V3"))
 (segment (start 102.5 58) (end 109.05 58) (width 0.2) (layer "B.Cu") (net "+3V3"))
 (segment (start 153.35 71.65) (end 154.525 72.825) (width 0.2) (layer "B.Cu") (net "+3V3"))
 (segment (start 109.05 58) (end 110.45 59.4) (width 0.2) (layer "B.Cu") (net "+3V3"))
 (segment (start 177 47.5) (end 188 47.5) (width 0.2) (layer "B.Cu") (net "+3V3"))
 (segment (start 164.275 72.825) (end 165.45 71.65) (width 0.2) (layer "B.Cu") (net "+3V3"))
 (segment (start 188 47.5) (end 188 66.5) (width 0.2) (layer "B.Cu") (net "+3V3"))
 (segment (start 188 66.5) (end 185.35 69.15) (width 0.2) (layer "B.Cu") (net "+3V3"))
 (segment (start 158.025 70.475) (end 156.85 71.65) (width 0.2) (layer "B.Cu") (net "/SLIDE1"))
 (segment (start 189.5 45.16) (end 189.5 67) (width 0.2) (layer "B.Cu") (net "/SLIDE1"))
 (segment (start 186.025 70.475) (end 158.025 70.475) (width 0.2) (layer "B.Cu") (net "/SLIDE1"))
 (segment (start 189.5 67) (end 186.025 70.475) (width 0.2) (layer "B.Cu") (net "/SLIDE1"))
 (segment (start 192.24 42.42) (end 189.5 45.16) (width 0.2) (layer "B.Cu") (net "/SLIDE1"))
 (segment (start 177 55.12) (end 142.08 55.12) (width 0.2) (layer "B.Cu") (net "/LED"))
 (segment (start 142.08 55.12) (end 138.1 59.1) (width 0.2) (layer "B.Cu") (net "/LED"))
 (segment (start 190.5 68) (end 186.85 71.65) (width 0.2) (layer "B.Cu") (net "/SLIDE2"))
 (segment (start 186.85 71.65) (end 168.95 71.65) (width 0.2) (layer "B.Cu") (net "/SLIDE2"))
 (segment (start 190.5 46.7) (end 190.5 68) (width 0.2) (layer "B.Cu") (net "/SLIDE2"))
 (segment (start 192.24 44.96) (end 190.5 46.7) (width 0.2) (layer "B.Cu") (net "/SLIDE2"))
 (segment (start 123.2547 60.5547) (end 141.2547 60.5547) (width 0.2) (layer "B.Cu") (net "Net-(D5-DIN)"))
 (segment (start 141.2547 60.5547) (end 143 62.3) (width 0.2) (layer "B.Cu") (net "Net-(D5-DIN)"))
 (segment (start 122.1 59.4) (end 123.2547 60.5547) (width 0.2) (layer "B.Cu") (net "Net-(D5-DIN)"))
 (segment (start 113 62.5) (end 113.5 62.5) (width 0.2) (layer "B.Cu") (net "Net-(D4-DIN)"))
 (segment (start 115 61) (end 125.4 61) (width 0.2) (layer "B.Cu") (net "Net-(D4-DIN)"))
 (segment (start 111.5 61) (end 113 62.5) (width 0.2) (layer "B.Cu") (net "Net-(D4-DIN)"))
 (segment (start 113.5 62.5) (end 115 61) (width 0.2) (layer "B.Cu") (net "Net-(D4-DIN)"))
 (segment (start 105.55 59.4) (end 107.15 61) (width 0.2) (layer "B.Cu") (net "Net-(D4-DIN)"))
 (segment (start 107.15 61) (end 111.5 61) (width 0.2) (layer "B.Cu") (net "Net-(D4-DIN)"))
 (segment (start 125.4 61) (end 127 62.6) (width 0.2) (layer "B.Cu") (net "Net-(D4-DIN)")))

